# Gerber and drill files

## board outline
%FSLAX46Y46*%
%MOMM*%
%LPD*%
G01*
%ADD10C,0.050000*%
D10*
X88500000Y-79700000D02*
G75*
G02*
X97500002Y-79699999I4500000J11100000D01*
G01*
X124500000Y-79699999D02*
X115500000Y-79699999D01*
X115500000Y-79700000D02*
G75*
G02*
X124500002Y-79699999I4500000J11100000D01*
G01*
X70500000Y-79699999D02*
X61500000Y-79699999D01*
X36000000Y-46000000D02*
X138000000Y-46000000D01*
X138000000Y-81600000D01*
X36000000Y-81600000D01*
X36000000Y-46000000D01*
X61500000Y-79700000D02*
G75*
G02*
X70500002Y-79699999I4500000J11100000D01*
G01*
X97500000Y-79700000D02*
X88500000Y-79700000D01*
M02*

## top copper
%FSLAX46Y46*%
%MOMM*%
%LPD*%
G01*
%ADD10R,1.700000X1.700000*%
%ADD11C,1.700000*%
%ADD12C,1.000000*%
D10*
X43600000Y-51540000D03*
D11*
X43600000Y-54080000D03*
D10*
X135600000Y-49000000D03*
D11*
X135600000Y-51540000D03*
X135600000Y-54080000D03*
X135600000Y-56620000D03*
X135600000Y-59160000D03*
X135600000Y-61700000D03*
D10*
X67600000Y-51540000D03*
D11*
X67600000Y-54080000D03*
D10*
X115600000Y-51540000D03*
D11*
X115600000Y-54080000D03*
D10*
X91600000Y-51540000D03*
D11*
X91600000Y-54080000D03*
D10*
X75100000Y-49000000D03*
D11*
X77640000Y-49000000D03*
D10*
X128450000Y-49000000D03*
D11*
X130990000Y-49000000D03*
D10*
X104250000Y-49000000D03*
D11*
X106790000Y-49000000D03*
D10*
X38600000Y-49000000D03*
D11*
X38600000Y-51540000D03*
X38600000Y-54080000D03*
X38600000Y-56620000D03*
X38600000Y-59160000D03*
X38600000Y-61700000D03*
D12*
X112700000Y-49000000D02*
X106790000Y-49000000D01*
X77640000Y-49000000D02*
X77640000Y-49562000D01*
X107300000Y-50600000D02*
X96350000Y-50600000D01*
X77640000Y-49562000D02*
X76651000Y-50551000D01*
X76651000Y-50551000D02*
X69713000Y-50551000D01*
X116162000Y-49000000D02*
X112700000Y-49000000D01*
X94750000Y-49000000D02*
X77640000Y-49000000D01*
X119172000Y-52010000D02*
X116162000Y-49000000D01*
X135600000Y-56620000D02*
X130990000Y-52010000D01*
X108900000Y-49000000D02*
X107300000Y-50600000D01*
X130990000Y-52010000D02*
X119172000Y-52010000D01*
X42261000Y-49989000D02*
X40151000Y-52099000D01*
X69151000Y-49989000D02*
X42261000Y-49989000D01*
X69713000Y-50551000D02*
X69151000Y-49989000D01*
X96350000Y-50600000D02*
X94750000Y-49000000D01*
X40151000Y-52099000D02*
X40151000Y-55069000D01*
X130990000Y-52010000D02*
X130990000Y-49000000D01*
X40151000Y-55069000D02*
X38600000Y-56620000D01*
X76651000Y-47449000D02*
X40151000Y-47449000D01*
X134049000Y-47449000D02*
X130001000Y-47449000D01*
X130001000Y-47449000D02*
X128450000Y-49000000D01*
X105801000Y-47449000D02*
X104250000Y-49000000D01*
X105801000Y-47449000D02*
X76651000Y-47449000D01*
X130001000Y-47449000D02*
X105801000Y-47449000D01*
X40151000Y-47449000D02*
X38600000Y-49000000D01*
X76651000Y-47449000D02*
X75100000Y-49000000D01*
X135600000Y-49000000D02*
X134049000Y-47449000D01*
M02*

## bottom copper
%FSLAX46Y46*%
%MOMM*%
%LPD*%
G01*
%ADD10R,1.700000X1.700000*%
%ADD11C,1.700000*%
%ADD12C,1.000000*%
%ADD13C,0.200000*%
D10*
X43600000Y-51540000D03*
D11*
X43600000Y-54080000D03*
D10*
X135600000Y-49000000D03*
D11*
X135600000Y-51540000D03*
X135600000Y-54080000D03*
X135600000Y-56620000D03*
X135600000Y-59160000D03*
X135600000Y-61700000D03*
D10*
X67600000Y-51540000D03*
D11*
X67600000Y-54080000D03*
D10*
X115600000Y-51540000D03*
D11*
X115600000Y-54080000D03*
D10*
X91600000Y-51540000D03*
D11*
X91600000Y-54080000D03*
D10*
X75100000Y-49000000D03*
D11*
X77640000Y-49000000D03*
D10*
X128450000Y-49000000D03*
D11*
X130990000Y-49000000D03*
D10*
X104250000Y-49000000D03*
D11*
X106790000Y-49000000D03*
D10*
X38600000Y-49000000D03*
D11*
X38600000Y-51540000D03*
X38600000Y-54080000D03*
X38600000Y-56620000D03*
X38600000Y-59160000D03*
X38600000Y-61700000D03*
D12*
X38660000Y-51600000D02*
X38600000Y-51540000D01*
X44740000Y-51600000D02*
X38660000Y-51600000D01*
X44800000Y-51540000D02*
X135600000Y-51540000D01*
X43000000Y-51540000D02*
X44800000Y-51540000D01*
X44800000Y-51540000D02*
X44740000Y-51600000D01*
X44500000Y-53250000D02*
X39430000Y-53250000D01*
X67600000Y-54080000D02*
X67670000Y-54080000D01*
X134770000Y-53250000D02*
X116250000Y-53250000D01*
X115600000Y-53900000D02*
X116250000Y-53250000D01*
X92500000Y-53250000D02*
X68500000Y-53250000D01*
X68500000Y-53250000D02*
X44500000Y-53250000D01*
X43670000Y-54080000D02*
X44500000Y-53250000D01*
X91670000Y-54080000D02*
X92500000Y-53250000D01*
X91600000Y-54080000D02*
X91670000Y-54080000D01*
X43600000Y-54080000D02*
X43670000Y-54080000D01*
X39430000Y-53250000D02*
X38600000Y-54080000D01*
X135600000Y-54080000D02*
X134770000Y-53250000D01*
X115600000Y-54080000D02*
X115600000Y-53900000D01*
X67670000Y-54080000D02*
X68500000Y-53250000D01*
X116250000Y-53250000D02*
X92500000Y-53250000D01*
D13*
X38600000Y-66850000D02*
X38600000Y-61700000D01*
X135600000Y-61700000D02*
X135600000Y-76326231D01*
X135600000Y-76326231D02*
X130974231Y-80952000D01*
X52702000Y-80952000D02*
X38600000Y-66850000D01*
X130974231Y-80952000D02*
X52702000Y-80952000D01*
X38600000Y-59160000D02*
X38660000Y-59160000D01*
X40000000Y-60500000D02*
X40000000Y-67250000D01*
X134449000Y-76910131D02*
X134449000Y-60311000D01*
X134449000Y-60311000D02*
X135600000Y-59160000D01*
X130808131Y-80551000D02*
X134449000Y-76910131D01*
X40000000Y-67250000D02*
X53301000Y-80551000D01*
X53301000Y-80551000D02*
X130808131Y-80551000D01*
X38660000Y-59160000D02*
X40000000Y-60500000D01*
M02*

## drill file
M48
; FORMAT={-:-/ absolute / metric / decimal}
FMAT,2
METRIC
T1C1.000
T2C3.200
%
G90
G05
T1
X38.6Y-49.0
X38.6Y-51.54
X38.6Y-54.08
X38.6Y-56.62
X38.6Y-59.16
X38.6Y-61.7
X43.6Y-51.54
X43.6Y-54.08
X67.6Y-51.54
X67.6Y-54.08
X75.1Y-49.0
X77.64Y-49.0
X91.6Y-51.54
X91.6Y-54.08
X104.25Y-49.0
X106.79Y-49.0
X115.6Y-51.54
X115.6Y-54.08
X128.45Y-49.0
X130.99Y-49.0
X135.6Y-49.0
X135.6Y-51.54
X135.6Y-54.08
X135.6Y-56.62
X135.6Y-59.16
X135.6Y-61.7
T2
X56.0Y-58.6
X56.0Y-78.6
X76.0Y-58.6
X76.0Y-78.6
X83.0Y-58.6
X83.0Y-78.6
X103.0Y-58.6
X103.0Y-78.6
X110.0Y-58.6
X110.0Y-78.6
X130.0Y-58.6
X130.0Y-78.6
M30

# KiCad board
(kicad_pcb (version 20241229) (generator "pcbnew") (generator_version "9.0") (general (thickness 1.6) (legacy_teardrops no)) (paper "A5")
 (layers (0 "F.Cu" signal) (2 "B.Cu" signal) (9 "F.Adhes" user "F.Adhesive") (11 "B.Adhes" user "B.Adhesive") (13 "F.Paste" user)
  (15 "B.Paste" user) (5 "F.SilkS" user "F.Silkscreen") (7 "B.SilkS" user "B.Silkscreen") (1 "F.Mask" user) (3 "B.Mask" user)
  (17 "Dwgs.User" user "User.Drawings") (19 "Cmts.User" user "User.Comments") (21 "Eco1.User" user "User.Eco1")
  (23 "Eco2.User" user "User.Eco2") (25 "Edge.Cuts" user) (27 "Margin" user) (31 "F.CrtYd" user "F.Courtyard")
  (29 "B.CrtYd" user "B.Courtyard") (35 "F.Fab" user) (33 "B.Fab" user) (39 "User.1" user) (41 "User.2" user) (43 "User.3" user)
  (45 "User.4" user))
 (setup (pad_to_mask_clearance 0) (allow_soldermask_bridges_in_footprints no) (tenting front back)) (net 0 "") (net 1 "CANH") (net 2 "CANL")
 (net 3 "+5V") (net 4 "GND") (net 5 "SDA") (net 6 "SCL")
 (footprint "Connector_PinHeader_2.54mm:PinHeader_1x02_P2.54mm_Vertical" (layer "F.Cu") (at 43.6 51.54)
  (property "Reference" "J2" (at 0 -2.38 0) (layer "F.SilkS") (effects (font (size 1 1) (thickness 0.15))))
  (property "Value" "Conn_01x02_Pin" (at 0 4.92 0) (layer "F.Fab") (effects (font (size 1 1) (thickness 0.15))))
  (pad "1" thru_hole rect (at 0 0) (size 1.7 1.7) (drill 1) (layers "*.Cu" "*.Mask") (remove_unused_layers no) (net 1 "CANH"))
  (pad "2" thru_hole circle (at 0 2.54) (size 1.7 1.7) (drill 1) (layers "*.Cu" "*.Mask") (remove_unused_layers no) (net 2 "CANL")))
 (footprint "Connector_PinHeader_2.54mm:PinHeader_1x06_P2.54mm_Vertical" (layer "F.Cu") (at 135.6 49)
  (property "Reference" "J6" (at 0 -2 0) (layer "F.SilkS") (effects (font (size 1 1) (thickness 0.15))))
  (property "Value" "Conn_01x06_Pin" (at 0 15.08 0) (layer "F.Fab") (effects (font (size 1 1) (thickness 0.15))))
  (pad "1" thru_hole rect (at 0 0) (size 1.7 1.7) (drill 1) (layers "*.Cu" "*.Mask") (remove_unused_layers no) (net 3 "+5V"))
  (pad "2" thru_hole circle (at 0 2.54) (size 1.7 1.7) (drill 1) (layers "*.Cu" "*.Mask") (remove_unused_layers no) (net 1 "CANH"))
  (pad "3" thru_hole circle (at 0 5.08) (size 1.7 1.7) (drill 1) (layers "*.Cu" "*.Mask") (remove_unused_layers no) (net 2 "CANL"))
  (pad "4" thru_hole circle (at 0 7.62) (size 1.7 1.7) (drill 1) (layers "*.Cu" "*.Mask") (remove_unused_layers no) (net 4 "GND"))
  (pad "5" thru_hole circle (at 0 10.16) (size 1.7 1.7) (drill 1) (layers "*.Cu" "*.Mask") (remove_unused_layers no) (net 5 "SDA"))
  (pad "6" thru_hole circle (at 0 12.7) (size 1.7 1.7) (drill 1) (layers "*.Cu" "*.Mask") (remove_unused_layers no) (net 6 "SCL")))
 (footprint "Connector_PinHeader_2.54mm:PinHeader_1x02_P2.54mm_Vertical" (layer "F.Cu") (at 67.6 51.54)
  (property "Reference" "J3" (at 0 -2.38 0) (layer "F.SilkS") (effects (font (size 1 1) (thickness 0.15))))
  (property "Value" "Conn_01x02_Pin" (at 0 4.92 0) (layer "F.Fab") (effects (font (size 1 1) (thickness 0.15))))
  (pad "1" thru_hole rect (at 0 0) (size 1.7 1.7) (drill 1) (layers "*.Cu" "*.Mask") (remove_unused_layers no) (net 1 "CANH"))
  (pad "2" thru_hole circle (at 0 2.54) (size 1.7 1.7) (drill 1) (layers "*.Cu" "*.Mask") (remove_unused_layers no) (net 2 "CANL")))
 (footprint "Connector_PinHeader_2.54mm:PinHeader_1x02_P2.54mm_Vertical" (layer "F.Cu") (at 115.6 51.54)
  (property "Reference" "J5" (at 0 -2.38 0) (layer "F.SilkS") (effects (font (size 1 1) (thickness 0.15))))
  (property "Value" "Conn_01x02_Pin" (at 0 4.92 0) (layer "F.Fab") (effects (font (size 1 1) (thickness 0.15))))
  (pad "1" thru_hole rect (at 0 0) (size 1.7 1.7) (drill 1) (layers "*.Cu" "*.Mask") (remove_unused_layers no) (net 1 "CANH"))
  (pad "2" thru_hole circle (at 0 2.54) (size 1.7 1.7) (drill 1) (layers "*.Cu" "*.Mask") (remove_unused_layers no) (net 2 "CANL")))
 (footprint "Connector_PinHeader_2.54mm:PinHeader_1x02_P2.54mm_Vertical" (layer "F.Cu") (at 91.6 51.54)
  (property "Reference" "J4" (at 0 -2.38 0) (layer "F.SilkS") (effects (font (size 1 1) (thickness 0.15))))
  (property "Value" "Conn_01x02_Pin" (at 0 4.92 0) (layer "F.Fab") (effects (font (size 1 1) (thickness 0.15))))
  (pad "1" thru_hole rect (at 0 0) (size 1.7 1.7) (drill 1) (layers "*.Cu" "*.Mask") (remove_unused_layers no) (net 1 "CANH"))
  (pad "2" thru_hole circle (at 0 2.54) (size 1.7 1.7) (drill 1) (layers "*.Cu" "*.Mask") (remove_unused_layers no) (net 2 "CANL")))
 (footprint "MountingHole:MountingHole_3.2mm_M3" (layer "B.Cu") (at 76 58.6 180)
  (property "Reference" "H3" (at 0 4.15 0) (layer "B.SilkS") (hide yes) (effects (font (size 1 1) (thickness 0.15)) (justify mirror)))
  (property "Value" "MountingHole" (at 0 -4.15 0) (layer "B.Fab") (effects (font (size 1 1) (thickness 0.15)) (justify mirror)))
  (pad "" np_thru_hole circle (at 0 0 180) (size 3.2 3.2) (drill 3.2) (layers "*.Cu" "*.Mask")))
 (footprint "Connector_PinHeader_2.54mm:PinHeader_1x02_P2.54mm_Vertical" (layer "B.Cu") (at 75.1 49 -90)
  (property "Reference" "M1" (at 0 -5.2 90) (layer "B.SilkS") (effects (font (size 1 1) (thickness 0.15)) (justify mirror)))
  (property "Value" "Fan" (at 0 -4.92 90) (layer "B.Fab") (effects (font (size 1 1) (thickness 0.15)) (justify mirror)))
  (pad "1" thru_hole rect (at 0 0 270) (size 1.7 1.7) (drill 1) (layers "*.Cu" "*.Mask") (remove_unused_layers no) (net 3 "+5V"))
  (pad "2" thru_hole circle (at 0 -2.54 270) (size 1.7 1.7) (drill 1) (layers "*.Cu" "*.Mask") (remove_unused_layers no) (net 4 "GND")))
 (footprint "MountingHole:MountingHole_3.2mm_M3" (layer "B.Cu") (at 76 78.6 180)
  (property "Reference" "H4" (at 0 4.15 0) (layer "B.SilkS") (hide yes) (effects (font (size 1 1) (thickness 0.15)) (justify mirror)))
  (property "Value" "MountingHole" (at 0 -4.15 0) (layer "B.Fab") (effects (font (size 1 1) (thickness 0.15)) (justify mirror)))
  (pad "" np_thru_hole circle (at 0 0 180) (size 3.2 3.2) (drill 3.2) (layers "*.Cu" "*.Mask")))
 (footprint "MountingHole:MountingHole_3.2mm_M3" (layer "B.Cu") (at 83 78.6 180)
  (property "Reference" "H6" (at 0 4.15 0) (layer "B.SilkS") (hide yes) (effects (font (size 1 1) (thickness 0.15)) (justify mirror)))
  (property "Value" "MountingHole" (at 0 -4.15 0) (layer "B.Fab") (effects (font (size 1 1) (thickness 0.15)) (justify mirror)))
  (pad "" np_thru_hole circle (at 0 0 180) (size 3.2 3.2) (drill 3.2) (layers "*.Cu" "*.Mask")))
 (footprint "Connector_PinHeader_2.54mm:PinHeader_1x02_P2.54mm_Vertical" (layer "B.Cu") (at 128.45 49 -90)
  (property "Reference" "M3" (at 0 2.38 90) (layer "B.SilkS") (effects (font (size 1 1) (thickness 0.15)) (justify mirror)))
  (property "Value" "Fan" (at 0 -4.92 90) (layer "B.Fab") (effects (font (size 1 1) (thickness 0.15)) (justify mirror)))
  (pad "1" thru_hole rect (at 0 0 270) (size 1.7 1.7) (drill 1) (layers "*.Cu" "*.Mask") (remove_unused_layers no) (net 3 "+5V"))
  (pad "2" thru_hole circle (at 0 -2.54 270) (size 1.7 1.7) (drill 1) (layers "*.Cu" "*.Mask") (remove_unused_layers no) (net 4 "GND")))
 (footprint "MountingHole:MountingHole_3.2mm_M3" (layer "B.Cu") (at 130 78.6 180)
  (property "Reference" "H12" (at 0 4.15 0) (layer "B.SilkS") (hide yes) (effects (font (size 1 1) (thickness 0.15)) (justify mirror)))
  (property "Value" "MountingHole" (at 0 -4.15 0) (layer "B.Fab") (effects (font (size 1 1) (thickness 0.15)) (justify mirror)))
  (pad "" np_thru_hole circle (at 0 0 180) (size 3.2 3.2) (drill 3.2) (layers "*.Cu" "*.Mask")))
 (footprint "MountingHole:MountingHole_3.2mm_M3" (layer "B.Cu") (at 103 78.6 180)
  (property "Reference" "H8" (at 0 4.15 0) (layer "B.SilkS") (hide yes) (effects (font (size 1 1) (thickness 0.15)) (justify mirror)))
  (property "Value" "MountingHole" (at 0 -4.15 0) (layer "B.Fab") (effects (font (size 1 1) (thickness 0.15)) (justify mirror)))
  (pad "" np_thru_hole circle (at 0 0 180) (size 3.2 3.2) (drill 3.2) (layers "*.Cu" "*.Mask")))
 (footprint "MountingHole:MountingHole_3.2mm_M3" (layer "B.Cu") (at 56 78.6 180)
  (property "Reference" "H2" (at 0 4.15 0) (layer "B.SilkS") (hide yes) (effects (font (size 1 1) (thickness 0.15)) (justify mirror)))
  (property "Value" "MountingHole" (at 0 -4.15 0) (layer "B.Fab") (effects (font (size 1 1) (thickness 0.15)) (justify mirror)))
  (pad "" np_thru_hole circle (at 0 0 180) (size 3.2 3.2) (drill 3.2) (layers "*.Cu" "*.Mask")))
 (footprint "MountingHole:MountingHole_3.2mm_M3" (layer "B.Cu") (at 110 78.6 180)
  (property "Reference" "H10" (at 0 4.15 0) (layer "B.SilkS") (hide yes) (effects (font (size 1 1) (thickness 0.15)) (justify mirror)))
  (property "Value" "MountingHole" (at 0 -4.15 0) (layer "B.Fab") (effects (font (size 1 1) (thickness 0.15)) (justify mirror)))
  (pad "" np_thru_hole circle (at 0 0 180) (size 3.2 3.2) (drill 3.2) (layers "*.Cu" "*.Mask")))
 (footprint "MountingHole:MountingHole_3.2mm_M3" (layer "B.Cu") (at 110 58.6 180)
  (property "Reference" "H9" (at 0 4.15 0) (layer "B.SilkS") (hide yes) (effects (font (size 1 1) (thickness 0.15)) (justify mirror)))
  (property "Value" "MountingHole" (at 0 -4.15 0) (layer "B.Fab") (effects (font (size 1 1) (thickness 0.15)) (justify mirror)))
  (pad "" np_thru_hole circle (at 0 0 180) (size 3.2 3.2) (drill 3.2) (layers "*.Cu" "*.Mask")))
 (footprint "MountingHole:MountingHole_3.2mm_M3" (layer "B.Cu") (at 103 58.6 180)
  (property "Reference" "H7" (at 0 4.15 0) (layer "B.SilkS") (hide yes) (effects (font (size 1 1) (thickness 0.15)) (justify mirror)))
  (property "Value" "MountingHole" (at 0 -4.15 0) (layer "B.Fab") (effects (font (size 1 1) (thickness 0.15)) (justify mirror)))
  (pad "" np_thru_hole circle (at 0 0 180) (size 3.2 3.2) (drill 3.2) (layers "*.Cu" "*.Mask")))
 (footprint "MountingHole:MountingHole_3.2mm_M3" (layer "B.Cu") (at 83 58.6 180)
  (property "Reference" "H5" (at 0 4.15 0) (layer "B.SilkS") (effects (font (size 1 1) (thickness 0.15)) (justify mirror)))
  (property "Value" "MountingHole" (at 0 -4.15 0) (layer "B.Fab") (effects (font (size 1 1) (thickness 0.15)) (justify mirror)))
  (pad "" np_thru_hole circle (at 0 0 180) (size 3.2 3.2) (drill 3.2) (layers "*.Cu" "*.Mask")))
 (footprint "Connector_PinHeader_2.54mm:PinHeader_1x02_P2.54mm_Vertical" (layer "B.Cu") (at 104.25 49 -90)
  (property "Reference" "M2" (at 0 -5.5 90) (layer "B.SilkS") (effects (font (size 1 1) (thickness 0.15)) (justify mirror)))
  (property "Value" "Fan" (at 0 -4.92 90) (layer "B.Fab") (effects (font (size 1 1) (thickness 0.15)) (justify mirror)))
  (pad "1" thru_hole rect (at 0 0 270) (size 1.7 1.7) (drill 1) (layers "*.Cu" "*.Mask") (remove_unused_layers no) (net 3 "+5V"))
  (pad "2" thru_hole circle (at 0 -2.54 270) (size 1.7 1.7) (drill 1) (layers "*.Cu" "*.Mask") (remove_unused_layers no) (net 4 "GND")))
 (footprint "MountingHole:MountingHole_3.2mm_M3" (layer "B.Cu") (at 130 58.6 180)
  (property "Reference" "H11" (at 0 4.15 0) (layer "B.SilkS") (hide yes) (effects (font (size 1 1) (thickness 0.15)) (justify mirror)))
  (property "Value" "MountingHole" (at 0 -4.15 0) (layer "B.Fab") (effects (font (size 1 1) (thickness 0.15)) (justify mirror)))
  (pad "" np_thru_hole circle (at 0 0 180) (size 3.2 3.2) (drill 3.2) (layers "*.Cu" "*.Mask")))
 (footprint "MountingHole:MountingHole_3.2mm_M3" (layer "B.Cu") (at 56 58.6 180)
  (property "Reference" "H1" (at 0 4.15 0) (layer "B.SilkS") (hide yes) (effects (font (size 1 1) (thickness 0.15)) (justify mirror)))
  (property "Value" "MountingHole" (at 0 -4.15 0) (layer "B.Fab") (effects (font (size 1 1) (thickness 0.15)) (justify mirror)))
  (pad "" np_thru_hole circle (at 0 0 180) (size 3.2 3.2) (drill 3.2) (layers "*.Cu" "*.Mask")))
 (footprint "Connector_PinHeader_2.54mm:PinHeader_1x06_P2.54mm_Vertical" (layer "B.Cu") (at 38.6 49 180)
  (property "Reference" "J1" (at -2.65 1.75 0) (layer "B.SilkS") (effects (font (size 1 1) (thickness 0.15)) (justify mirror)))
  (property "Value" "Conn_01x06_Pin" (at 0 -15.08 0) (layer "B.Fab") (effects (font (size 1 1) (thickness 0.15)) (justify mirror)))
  (pad "1" thru_hole rect (at 0 0 180) (size 1.7 1.7) (drill 1) (layers "*.Cu" "*.Mask") (remove_unused_layers no) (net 3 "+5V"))
  (pad "2" thru_hole circle (at 0 -2.54 180) (size 1.7 1.7) (drill 1) (layers "*.Cu" "*.Mask") (remove_unused_layers no) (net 1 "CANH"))
  (pad "3" thru_hole circle (at 0 -5.08 180) (size 1.7 1.7) (drill 1) (layers "*.Cu" "*.Mask") (remove_unused_layers no) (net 2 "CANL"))
  (pad "4" thru_hole circle (at 0 -7.62 180) (size 1.7 1.7) (drill 1) (layers "*.Cu" "*.Mask") (remove_unused_layers no) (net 4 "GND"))
  (pad "5" thru_hole circle (at 0 -10.16 180) (size 1.7 1.7) (drill 1) (layers "*.Cu" "*.Mask") (remove_unused_layers no) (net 5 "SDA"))
  (pad "6" thru_hole circle (at 0 -12.7 180) (size 1.7 1.7) (drill 1) (layers "*.Cu" "*.Mask") (remove_unused_layers no) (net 6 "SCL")))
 (gr_arc (start 88.5 79.7) (mid 92.999999 56.622521) (end 97.500002 79.699999) (stroke (width 0.05) (type default)) (layer "Edge.Cuts"))
 (gr_line (start 124.5 79.699999) (end 115.5 79.699999) (stroke (width 0.05) (type default)) (layer "Edge.Cuts"))
 (gr_arc (start 115.5 79.7) (mid 119.999999 56.622521) (end 124.500002 79.699999) (stroke (width 0.05) (type default)) (layer "Edge.Cuts"))
 (gr_line (start 70.5 79.699999) (end 61.5 79.699999) (stroke (width 0.05) (type default)) (layer "Edge.Cuts"))
 (gr_rect (start 36 46) (end 138 81.6) (stroke (width 0.05) (type solid)) (fill no) (layer "Edge.Cuts"))
 (gr_arc (start 61.5 79.7) (mid 65.999999 56.622521) (end 70.500002 79.699999) (stroke (width 0.05) (type default)) (layer "Edge.Cuts"))
 (gr_line (start 97.5 79.7) (end 88.5 79.7) (stroke (width 0.05) (type default)) (layer "Edge.Cuts"))
 (segment (start 38.66 51.6) (end 38.6 51.54) (width 1) (layer "B.Cu") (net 1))
 (segment (start 44.74 51.6) (end 38.66 51.6) (width 1) (layer "B.Cu") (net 1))
 (segment (start 44.8 51.54) (end 135.6 51.54) (width 1) (layer "B.Cu") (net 1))
 (segment (start 43 51.54) (end 44.8 51.54) (width 1) (layer "B.Cu") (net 1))
 (segment (start 44.8 51.54) (end 44.74 51.6) (width 1) (layer "B.Cu") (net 1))
 (segment (start 44.5 53.25) (end 39.43 53.25) (width 1) (layer "B.Cu") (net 2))
 (segment (start 67.6 54.08) (end 67.67 54.08) (width 1) (layer "B.Cu") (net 2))
 (segment (start 134.77 53.25) (end 116.25 53.25) (width 1) (layer "B.Cu") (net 2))
 (segment (start 115.6 53.9) (end 116.25 53.25) (width 1) (layer "B.Cu") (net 2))
 (segment (start 92.5 53.25) (end 68.5 53.25) (width 1) (layer "B.Cu") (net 2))
 (segment (start 68.5 53.25) (end 44.5 53.25) (width 1) (layer "B.Cu") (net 2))
 (segment (start 43.67 54.08) (end 44.5 53.25) (width 1) (layer "B.Cu") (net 2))
 (segment (start 91.67 54.08) (end 92.5 53.25) (width 1) (layer "B.Cu") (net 2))
 (segment (start 91.6 54.08) (end 91.67 54.08) (width 1) (layer "B.Cu") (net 2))
 (segment (start 43.6 54.08) (end 43.67 54.08) (width 1) (layer "B.Cu") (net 2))
 (segment (start 39.43 53.25) (end 38.6 54.08) (width 1) (layer "B.Cu") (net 2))
 (segment (start 135.6 54.08) (end 134.77 53.25) (width 1) (layer "B.Cu") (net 2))
 (segment (start 115.6 54.08) (end 115.6 53.9) (width 1) (layer "B.Cu") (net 2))
 (segment (start 67.67 54.08) (end 68.5 53.25) (width 1) (layer "B.Cu") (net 2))
 (segment (start 116.25 53.25) (end 92.5 53.25) (width 1) (layer "B.Cu") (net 2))
 (segment (start 38.6 66.85) (end 38.6 61.7) (width 0.2) (layer "B.Cu") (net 6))
 (segment (start 135.6 61.7) (end 135.6 76.326231) (width 0.2) (layer "B.Cu") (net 6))
 (segment (start 135.6 76.326231) (end 130.974231 80.952) (width 0.2) (layer "B.Cu") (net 6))
 (segment (start 52.702 80.952) (end 38.6 66.85) (width 0.2) (layer "B.Cu") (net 6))
 (segment (start 130.974231 80.952) (end 52.702 80.952) (width 0.2) (layer "B.Cu") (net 6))
 (segment (start 38.6 59.16) (end 38.66 59.16) (width 0.2) (layer "B.Cu") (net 5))
 (segment (start 40 60.5) (end 40 67.25) (width 0.2) (layer "B.Cu") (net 5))
 (segment (start 134.449 76.910131) (end 134.449 60.311) (width 0.2) (layer "B.Cu") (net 5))
 (segment (start 134.449 60.311) (end 135.6 59.16) (width 0.2) (layer "B.Cu") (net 5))
 (segment (start 130.808131 80.551) (end 134.449 76.910131) (width 0.2) (layer "B.Cu") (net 5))
 (segment (start 40 67.25) (end 53.301 80.551) (width 0.2) (layer "B.Cu") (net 5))
 (segment (start 53.301 80.551) (end 130.808131 80.551) (width 0.2) (layer "B.Cu") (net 5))
 (segment (start 38.66 59.16) (end 40 60.5) (width 0.2) (layer "B.Cu") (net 5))
 (segment (start 112.7 49) (end 106.79 49) (width 1) (layer "F.Cu") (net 4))
 (segment (start 77.64 49) (end 77.64 49.562) (width 1) (layer "F.Cu") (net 4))
 (segment (start 107.3 50.6) (end 96.35 50.6) (width 1) (layer "F.Cu") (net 4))
 (segment (start 77.64 49.562) (end 76.651 50.551) (width 1) (layer "F.Cu") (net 4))
 (segment (start 76.651 50.551) (end 69.713 50.551) (width 1) (layer "F.Cu") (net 4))
 (segment (start 116.162 49) (end 112.7 49) (width 1) (layer "F.Cu") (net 4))
 (segment (start 94.75 49) (end 77.64 49) (width 1) (layer "F.Cu") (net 4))
 (segment (start 119.172 52.01) (end 116.162 49) (width 1) (layer "F.Cu") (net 4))
 (segment (start 135.6 56.62) (end 130.99 52.01) (width 1) (layer "F.Cu") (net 4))
 (segment (start 108.9 49) (end 107.3 50.6) (width 1) (layer "F.Cu") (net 4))
 (segment (start 130.99 52.01) (end 119.172 52.01) (width 1) (layer "F.Cu") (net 4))
 (segment (start 42.261 49.989) (end 40.151 52.099) (width 1) (layer "F.Cu") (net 4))
 (segment (start 69.151 49.989) (end 42.261 49.989) (width 1) (layer "F.Cu") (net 4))
 (segment (start 69.713 50.551) (end 69.151 49.989) (width 1) (layer "F.Cu") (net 4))
 (segment (start 96.35 50.6) (end 94.75 49) (width 1) (layer "F.Cu") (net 4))
 (segment (start 40.151 52.099) (end 40.151 55.069) (width 1) (layer "F.Cu") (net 4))
 (segment (start 130.99 52.01) (end 130.99 49) (width 1) (layer "F.Cu") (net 4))
 (segment (start 40.151 55.069) (end 38.6 56.62) (width 1) (layer "F.Cu") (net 4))
 (segment (start 76.651 47.449) (end 40.151 47.449) (width 1) (layer "F.Cu") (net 3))
 (segment (start 134.049 47.449) (end 130.001 47.449) (width 1) (layer "F.Cu") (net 3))
 (segment (start 130.001 47.449) (end 128.45 49) (width 1) (layer "F.Cu") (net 3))
 (segment (start 105.801 47.449) (end 104.25 49) (width 1) (layer "F.Cu") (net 3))
 (segment (start 105.801 47.449) (end 76.651 47.449) (width 1) (layer "F.Cu") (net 3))
 (segment (start 130.001 47.449) (end 105.801 47.449) (width 1) (layer "F.Cu") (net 3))
 (segment (start 40.151 47.449) (end 38.6 49) (width 1) (layer "F.Cu") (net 3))
 (segment (start 76.651 47.449) (end 75.1 49) (width 1) (layer "F.Cu") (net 3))
 (segment (start 135.6 49) (end 134.049 47.449) (width 1) (layer "F.Cu") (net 3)))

